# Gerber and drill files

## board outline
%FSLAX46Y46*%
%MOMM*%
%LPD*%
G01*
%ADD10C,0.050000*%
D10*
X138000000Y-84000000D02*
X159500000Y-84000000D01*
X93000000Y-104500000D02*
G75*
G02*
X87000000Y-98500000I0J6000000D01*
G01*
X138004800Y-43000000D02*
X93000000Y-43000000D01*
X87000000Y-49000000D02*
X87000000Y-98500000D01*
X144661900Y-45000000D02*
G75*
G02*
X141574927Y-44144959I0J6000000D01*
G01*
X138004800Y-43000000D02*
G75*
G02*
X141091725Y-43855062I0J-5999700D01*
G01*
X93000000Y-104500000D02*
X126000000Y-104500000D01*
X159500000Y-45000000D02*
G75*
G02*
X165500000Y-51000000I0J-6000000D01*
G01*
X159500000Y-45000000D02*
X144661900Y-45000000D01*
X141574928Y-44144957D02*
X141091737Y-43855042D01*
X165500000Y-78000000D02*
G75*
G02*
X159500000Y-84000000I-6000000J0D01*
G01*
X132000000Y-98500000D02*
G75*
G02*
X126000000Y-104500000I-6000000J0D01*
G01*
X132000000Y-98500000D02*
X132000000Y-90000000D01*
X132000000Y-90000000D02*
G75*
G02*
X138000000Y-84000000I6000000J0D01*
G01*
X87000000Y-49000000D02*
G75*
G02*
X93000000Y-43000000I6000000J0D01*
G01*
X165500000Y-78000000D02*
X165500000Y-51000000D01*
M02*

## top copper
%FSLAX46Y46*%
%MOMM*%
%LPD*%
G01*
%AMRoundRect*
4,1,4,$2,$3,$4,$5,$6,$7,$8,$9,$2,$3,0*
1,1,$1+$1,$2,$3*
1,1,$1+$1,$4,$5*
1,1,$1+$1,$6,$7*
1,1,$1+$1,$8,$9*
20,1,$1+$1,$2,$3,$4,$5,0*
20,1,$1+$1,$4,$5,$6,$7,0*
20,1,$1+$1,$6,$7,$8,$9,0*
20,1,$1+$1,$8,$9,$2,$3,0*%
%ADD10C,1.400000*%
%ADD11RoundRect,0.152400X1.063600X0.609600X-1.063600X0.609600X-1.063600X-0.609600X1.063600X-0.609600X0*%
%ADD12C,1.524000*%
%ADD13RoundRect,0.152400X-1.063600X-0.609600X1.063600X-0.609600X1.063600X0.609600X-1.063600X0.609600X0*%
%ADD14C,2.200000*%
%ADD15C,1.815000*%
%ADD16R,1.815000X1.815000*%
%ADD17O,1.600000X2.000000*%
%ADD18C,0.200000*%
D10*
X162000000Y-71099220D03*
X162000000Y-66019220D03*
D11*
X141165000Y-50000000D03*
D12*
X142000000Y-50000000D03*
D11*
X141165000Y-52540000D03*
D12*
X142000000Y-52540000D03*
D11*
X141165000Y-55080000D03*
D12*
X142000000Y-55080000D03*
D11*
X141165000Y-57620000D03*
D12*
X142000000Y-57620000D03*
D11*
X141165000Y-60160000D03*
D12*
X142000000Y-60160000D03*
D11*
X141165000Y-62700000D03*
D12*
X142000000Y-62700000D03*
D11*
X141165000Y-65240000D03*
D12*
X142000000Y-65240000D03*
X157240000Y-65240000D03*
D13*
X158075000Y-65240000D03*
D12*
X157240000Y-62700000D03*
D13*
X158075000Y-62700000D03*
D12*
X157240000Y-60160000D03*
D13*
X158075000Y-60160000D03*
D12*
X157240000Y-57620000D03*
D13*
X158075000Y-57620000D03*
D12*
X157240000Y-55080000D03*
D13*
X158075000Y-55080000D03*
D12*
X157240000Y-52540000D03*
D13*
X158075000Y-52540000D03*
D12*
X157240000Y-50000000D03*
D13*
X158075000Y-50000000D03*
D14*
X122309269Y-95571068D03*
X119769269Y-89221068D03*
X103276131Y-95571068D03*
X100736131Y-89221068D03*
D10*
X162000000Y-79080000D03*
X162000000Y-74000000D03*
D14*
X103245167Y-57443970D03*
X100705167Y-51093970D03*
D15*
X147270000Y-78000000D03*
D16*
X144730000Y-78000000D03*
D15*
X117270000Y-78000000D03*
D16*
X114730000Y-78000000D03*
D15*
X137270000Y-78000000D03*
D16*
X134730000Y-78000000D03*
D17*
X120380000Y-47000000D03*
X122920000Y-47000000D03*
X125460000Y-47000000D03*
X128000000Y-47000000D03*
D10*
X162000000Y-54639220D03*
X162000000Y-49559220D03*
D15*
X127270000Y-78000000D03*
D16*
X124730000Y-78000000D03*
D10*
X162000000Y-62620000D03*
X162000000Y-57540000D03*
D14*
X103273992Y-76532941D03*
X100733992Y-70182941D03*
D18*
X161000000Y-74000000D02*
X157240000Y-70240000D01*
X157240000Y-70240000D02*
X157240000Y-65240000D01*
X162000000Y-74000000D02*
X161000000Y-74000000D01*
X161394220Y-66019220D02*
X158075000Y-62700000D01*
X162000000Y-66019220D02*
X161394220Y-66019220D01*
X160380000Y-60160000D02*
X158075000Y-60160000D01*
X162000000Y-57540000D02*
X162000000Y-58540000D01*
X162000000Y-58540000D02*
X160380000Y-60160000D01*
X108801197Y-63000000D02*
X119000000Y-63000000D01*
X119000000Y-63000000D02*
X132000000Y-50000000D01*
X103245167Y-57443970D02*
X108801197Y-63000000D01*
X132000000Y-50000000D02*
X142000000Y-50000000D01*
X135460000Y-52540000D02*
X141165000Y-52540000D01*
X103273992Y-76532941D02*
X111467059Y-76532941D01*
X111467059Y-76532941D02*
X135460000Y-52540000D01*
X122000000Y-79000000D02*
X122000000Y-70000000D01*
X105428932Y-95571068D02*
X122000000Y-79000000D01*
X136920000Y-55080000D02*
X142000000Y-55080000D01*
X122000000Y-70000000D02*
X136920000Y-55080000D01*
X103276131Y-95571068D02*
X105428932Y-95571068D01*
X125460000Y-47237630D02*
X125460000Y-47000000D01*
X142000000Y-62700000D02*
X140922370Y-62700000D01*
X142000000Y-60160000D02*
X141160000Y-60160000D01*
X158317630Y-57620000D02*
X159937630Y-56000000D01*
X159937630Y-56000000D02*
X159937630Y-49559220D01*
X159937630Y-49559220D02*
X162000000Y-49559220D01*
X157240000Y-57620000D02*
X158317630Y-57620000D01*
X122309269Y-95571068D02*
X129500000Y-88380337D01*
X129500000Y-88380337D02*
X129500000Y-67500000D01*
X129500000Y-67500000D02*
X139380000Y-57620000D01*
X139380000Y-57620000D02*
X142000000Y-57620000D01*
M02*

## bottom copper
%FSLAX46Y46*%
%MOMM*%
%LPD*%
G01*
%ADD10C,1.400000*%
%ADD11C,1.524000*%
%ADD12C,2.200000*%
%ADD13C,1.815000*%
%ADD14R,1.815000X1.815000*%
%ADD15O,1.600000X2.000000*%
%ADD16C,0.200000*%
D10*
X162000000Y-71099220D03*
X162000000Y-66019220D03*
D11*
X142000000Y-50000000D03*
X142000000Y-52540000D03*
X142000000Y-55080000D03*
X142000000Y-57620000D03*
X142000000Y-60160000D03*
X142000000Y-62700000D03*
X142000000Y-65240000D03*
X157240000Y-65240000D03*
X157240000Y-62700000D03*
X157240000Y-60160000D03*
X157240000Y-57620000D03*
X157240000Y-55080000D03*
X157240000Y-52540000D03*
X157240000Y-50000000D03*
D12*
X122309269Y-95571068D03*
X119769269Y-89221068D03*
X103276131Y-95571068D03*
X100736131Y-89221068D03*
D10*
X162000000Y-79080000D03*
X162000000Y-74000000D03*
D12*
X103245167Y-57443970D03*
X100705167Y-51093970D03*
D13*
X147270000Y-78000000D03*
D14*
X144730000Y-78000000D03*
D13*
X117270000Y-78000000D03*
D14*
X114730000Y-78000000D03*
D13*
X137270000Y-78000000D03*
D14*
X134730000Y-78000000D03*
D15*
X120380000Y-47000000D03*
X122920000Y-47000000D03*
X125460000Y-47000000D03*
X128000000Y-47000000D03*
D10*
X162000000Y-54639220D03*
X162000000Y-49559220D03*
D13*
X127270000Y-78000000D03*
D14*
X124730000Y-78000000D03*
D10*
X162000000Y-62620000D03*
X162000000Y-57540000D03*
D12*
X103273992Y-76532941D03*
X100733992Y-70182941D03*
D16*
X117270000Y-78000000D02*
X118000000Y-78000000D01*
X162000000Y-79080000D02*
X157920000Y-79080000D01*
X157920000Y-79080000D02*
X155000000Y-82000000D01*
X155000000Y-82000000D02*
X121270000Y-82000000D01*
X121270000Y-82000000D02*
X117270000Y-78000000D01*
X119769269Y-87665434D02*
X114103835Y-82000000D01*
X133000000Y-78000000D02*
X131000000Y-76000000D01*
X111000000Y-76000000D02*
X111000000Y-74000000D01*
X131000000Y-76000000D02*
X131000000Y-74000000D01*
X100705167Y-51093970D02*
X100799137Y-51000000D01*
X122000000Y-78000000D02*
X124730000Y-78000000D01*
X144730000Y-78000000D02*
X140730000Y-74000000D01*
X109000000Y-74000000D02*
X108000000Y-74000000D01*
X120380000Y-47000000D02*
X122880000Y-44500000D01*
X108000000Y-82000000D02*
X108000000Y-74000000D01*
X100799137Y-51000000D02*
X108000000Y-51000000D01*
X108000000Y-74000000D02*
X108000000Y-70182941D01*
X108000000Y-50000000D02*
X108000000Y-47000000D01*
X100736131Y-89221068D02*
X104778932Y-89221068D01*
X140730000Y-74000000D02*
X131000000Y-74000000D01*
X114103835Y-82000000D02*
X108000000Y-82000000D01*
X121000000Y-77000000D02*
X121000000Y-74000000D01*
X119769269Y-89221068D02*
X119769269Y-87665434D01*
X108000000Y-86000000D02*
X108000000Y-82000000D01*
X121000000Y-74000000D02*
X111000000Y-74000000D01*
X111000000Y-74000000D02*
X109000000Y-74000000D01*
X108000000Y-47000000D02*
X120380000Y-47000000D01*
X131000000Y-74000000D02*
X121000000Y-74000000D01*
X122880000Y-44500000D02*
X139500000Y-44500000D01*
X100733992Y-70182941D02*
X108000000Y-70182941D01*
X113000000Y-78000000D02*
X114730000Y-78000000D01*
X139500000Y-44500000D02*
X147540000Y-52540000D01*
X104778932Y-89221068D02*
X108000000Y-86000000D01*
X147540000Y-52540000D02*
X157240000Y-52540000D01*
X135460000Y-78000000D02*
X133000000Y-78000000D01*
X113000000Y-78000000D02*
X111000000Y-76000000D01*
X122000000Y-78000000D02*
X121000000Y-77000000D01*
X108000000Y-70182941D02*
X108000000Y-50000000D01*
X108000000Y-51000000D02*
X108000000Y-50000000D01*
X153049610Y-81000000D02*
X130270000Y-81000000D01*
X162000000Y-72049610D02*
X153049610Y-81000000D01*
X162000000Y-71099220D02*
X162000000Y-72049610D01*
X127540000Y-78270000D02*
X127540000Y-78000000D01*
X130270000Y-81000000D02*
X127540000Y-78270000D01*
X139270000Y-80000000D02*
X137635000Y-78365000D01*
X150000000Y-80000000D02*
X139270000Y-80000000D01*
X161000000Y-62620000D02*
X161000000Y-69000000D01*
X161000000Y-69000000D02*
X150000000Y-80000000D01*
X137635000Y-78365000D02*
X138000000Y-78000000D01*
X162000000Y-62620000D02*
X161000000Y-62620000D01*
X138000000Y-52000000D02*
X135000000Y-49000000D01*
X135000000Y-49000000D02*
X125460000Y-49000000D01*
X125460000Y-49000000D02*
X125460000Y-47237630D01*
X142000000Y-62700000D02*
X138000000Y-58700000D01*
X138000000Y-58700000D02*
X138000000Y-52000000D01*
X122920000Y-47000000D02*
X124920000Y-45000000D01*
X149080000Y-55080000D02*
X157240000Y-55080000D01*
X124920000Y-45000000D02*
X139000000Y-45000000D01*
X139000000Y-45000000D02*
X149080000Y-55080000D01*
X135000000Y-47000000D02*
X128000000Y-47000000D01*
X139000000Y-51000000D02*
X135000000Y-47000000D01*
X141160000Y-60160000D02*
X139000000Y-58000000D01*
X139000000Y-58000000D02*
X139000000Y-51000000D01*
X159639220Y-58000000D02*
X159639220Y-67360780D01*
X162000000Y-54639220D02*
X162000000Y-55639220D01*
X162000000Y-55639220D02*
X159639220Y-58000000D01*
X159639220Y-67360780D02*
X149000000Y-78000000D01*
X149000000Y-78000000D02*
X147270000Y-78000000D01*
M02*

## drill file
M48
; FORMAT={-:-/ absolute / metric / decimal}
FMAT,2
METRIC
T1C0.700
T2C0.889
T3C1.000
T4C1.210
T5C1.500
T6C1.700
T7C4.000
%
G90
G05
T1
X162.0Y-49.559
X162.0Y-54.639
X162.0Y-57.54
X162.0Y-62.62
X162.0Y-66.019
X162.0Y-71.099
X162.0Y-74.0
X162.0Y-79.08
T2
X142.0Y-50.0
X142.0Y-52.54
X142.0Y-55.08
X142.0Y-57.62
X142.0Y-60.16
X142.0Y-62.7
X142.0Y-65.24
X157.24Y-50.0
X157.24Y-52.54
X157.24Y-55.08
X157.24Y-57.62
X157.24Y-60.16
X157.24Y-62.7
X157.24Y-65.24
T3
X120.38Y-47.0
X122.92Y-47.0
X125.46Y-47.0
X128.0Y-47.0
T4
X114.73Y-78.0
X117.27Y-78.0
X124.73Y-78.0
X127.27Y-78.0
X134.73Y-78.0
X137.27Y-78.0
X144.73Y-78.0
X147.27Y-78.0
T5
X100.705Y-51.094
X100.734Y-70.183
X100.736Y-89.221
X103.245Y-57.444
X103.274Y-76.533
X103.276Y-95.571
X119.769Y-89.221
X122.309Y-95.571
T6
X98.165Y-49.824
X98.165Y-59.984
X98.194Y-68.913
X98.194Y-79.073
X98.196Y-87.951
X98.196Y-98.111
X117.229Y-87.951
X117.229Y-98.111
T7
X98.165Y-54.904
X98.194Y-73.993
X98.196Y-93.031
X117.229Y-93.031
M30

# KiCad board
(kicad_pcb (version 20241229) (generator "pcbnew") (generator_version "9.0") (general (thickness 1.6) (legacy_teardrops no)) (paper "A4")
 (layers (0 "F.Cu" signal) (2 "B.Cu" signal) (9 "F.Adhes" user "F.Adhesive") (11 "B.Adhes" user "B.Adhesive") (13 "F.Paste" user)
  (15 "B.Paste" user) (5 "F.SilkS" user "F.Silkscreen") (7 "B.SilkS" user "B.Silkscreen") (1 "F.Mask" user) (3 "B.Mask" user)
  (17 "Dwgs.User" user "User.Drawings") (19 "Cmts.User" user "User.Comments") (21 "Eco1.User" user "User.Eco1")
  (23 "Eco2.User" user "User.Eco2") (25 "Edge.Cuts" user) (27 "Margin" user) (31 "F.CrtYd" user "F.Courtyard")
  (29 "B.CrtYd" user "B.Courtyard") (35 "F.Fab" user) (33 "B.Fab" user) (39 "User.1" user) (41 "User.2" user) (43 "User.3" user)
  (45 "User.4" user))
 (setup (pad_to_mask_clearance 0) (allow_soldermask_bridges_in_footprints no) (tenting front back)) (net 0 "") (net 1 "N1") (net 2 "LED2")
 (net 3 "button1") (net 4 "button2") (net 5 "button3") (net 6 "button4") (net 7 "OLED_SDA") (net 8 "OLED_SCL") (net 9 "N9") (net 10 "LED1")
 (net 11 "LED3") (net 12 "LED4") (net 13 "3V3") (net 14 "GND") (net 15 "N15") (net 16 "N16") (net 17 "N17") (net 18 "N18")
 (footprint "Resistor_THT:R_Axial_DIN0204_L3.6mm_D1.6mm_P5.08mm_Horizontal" (layer "F.Cu") (at 162 71.09922 90)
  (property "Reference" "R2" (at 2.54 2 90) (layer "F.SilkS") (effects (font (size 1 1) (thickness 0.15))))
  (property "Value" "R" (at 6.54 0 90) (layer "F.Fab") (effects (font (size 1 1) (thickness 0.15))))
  (pad "1" thru_hole circle (at 0 0 90) (size 1.4 1.4) (drill 0.7) (layers "*.Cu" "*.Mask") (remove_unused_layers no) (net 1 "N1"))
  (pad "2" thru_hole circle (at 5.08 0 90) (size 1.4 1.4) (drill 0.7) (layers "*.Cu" "*.Mask") (remove_unused_layers no) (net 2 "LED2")))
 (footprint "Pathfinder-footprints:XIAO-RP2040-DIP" (layer "F.Cu") (at 149.62 57.62)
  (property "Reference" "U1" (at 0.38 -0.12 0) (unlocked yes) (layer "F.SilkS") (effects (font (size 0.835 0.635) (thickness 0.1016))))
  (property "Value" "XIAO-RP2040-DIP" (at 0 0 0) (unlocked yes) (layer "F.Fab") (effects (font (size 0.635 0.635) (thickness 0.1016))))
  (pad "1" smd roundrect (at -8.455 -7.62 180) (size 2.432 1.524) (layers "F.Cu" "F.Mask") (roundrect_rratio 0.1) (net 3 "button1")
   (thermal_bridge_angle 45))
  (pad "1" thru_hole circle (at -7.62 -7.62 180) (size 1.524 1.524) (drill 0.889) (layers "*.Cu" "*.Mask") (remove_unused_layers no)
   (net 3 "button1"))
  (pad "2" smd roundrect (at -8.455 -5.08 180) (size 2.432 1.524) (layers "F.Cu" "F.Mask") (roundrect_rratio 0.1) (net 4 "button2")
   (thermal_bridge_angle 45))
  (pad "2" thru_hole circle (at -7.62 -5.08 180) (size 1.524 1.524) (drill 0.889) (layers "*.Cu" "*.Mask") (remove_unused_layers no)
   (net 4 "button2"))
  (pad "3" smd roundrect (at -8.455 -2.54 180) (size 2.432 1.524) (layers "F.Cu" "F.Mask") (roundrect_rratio 0.1) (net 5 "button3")
   (thermal_bridge_angle 45))
  (pad "3" thru_hole circle (at -7.62 -2.54 180) (size 1.524 1.524) (drill 0.889) (layers "*.Cu" "*.Mask") (remove_unused_layers no)
   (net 5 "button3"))
  (pad "4" smd roundrect (at -8.455 0 180) (size 2.432 1.524) (layers "F.Cu" "F.Mask") (roundrect_rratio 0.1) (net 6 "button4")
   (thermal_bridge_angle 45))
  (pad "4" thru_hole circle (at -7.62 0 180) (size 1.524 1.524) (drill 0.889) (layers "*.Cu" "*.Mask") (remove_unused_layers no)
   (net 6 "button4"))
  (pad "5" smd roundrect (at -8.455 2.54 180) (size 2.432 1.524) (layers "F.Cu" "F.Mask") (roundrect_rratio 0.1) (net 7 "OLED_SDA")
   (thermal_bridge_angle 45))
  (pad "5" thru_hole circle (at -7.62 2.54 180) (size 1.524 1.524) (drill 0.889) (layers "*.Cu" "*.Mask") (remove_unused_layers no)
   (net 7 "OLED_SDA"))
  (pad "6" smd roundrect (at -8.455 5.08 180) (size 2.432 1.524) (layers "F.Cu" "F.Mask") (roundrect_rratio 0.1) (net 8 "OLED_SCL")
   (thermal_bridge_angle 45))
  (pad "6" thru_hole circle (at -7.62 5.08 180) (size 1.524 1.524) (drill 0.889) (layers "*.Cu" "*.Mask") (remove_unused_layers no)
   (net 8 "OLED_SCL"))
  (pad "7" smd roundrect (at -8.455 7.62 180) (size 2.432 1.524) (layers "F.Cu" "F.Mask") (roundrect_rratio 0.1) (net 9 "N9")
   (thermal_bridge_angle 45))
  (pad "7" thru_hole circle (at -7.62 7.62 180) (size 1.524 1.524) (drill 0.889) (layers "*.Cu" "*.Mask") (remove_unused_layers no)
   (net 9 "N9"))
  (pad "8" thru_hole circle (at 7.62 7.62) (size 1.524 1.524) (drill 0.889) (layers "*.Cu" "*.Mask") (remove_unused_layers no)
   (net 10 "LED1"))
  (pad "8" smd roundrect (at 8.455 7.62) (size 2.432 1.524) (layers "F.Cu" "F.Mask") (roundrect_rratio 0.1) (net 10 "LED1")
   (thermal_bridge_angle 45))
  (pad "9" thru_hole circle (at 7.62 5.08) (size 1.524 1.524) (drill 0.889) (layers "*.Cu" "*.Mask") (remove_unused_layers no)
   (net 2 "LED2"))
  (pad "9" smd roundrect (at 8.455 5.08) (size 2.432 1.524) (layers "F.Cu" "F.Mask") (roundrect_rratio 0.1) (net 2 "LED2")
   (thermal_bridge_angle 45))
  (pad "10" thru_hole circle (at 7.62 2.54) (size 1.524 1.524) (drill 0.889) (layers "*.Cu" "*.Mask") (remove_unused_layers no)
   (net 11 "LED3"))
  (pad "10" smd roundrect (at 8.455 2.54) (size 2.432 1.524) (layers "F.Cu" "F.Mask") (roundrect_rratio 0.1) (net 11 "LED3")
   (thermal_bridge_angle 45))
  (pad "11" thru_hole circle (at 7.62 0) (size 1.524 1.524) (drill 0.889) (layers "*.Cu" "*.Mask") (remove_unused_layers no) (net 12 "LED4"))
  (pad "11" smd roundrect (at 8.455 0) (size 2.432 1.524) (layers "F.Cu" "F.Mask") (roundrect_rratio 0.1) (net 12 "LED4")
   (thermal_bridge_angle 45))
  (pad "12" thru_hole circle (at 7.62 -2.54) (size 1.524 1.524) (drill 0.889) (layers "*.Cu" "*.Mask") (remove_unused_layers no)
   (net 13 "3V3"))
  (pad "12" smd roundrect (at 8.455 -2.54) (size 2.432 1.524) (layers "F.Cu" "F.Mask") (roundrect_rratio 0.1) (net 13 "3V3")
   (thermal_bridge_angle 45))
  (pad "13" thru_hole circle (at 7.62 -5.08) (size 1.524 1.524) (drill 0.889) (layers "*.Cu" "*.Mask") (remove_unused_layers no)
   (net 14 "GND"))
  (pad "13" smd roundrect (at 8.455 -5.08) (size 2.432 1.524) (layers "F.Cu" "F.Mask") (roundrect_rratio 0.1) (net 14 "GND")
   (thermal_bridge_angle 45))
  (pad "14" thru_hole circle (at 7.62 -7.62) (size 1.524 1.524) (drill 0.889) (layers "*.Cu" "*.Mask") (remove_unused_layers no)
   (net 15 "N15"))
  (pad "14" smd roundrect (at 8.455 -7.62) (size 2.432 1.524) (layers "F.Cu" "F.Mask") (roundrect_rratio 0.1) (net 15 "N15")
   (thermal_bridge_angle 45)))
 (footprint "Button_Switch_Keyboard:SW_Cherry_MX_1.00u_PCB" (layer "F.Cu") (at 122.309269 95.571068 -90)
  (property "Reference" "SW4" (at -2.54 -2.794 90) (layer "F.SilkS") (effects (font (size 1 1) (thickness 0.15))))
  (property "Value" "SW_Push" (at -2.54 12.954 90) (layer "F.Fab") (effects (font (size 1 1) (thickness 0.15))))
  (pad "" np_thru_hole circle (at -7.62 5.08 270) (size 1.7 1.7) (drill 1.7) (layers "*.Cu" "*.Mask"))
  (pad "" np_thru_hole circle (at -2.54 5.08 270) (size 4 4) (drill 4) (layers "*.Cu" "*.Mask"))
  (pad "" np_thru_hole circle (at 2.54 5.08 270) (size 1.7 1.7) (drill 1.7) (layers "*.Cu" "*.Mask"))
  (pad "1" thru_hole circle (at 0 0 270) (size 2.2 2.2) (drill 1.5) (layers "*.Cu" "*.Mask") (remove_unused_layers no) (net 6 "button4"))
  (pad "2" thru_hole circle (at -6.35 2.54 270) (size 2.2 2.2) (drill 1.5) (layers "*.Cu" "*.Mask") (remove_unused_layers no) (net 14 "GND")))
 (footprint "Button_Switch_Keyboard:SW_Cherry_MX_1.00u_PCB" (layer "F.Cu") (at 103.276131 95.571068 -90)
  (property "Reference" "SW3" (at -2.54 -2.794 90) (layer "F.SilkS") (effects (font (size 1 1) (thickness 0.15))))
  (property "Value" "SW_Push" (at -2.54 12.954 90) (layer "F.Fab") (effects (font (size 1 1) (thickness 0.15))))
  (pad "" np_thru_hole circle (at -7.62 5.08 270) (size 1.7 1.7) (drill 1.7) (layers "*.Cu" "*.Mask"))
  (pad "" np_thru_hole circle (at -2.54 5.08 270) (size 4 4) (drill 4) (layers "*.Cu" "*.Mask"))
  (pad "" np_thru_hole circle (at 2.54 5.08 270) (size 1.7 1.7) (drill 1.7) (layers "*.Cu" "*.Mask"))
  (pad "1" thru_hole circle (at 0 0 270) (size 2.2 2.2) (drill 1.5) (layers "*.Cu" "*.Mask") (remove_unused_layers no) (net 5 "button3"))
  (pad "2" thru_hole circle (at -6.35 2.54 270) (size 2.2 2.2) (drill 1.5) (layers "*.Cu" "*.Mask") (remove_unused_layers no) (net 14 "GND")))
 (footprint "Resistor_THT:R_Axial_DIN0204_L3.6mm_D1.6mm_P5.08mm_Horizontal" (layer "F.Cu") (at 162 79.08 90)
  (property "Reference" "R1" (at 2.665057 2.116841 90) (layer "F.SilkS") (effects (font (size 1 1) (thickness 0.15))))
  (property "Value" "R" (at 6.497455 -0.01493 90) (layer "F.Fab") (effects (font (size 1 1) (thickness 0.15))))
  (pad "1" thru_hole circle (at 0 0 90) (size 1.4 1.4) (drill 0.7) (layers "*.Cu" "*.Mask") (remove_unused_layers no) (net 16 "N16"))
  (pad "2" thru_hole circle (at 5.08 0 90) (size 1.4 1.4) (drill 0.7) (layers "*.Cu" "*.Mask") (remove_unused_layers no) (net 10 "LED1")))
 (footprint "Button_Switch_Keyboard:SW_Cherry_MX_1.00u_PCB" (layer "F.Cu") (at 103.245167 57.44397 -90)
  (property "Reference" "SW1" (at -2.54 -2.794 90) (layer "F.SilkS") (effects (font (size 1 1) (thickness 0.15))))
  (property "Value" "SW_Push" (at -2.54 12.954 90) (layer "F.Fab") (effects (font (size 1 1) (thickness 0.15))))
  (pad "" np_thru_hole circle (at -7.62 5.08 270) (size 1.7 1.7) (drill 1.7) (layers "*.Cu" "*.Mask"))
  (pad "" np_thru_hole circle (at -2.54 5.08 270) (size 4 4) (drill 4) (layers "*.Cu" "*.Mask"))
  (pad "" np_thru_hole circle (at 2.54 5.08 270) (size 1.7 1.7) (drill 1.7) (layers "*.Cu" "*.Mask"))
  (pad "1" thru_hole circle (at 0 0 270) (size 2.2 2.2) (drill 1.5) (layers "*.Cu" "*.Mask") (remove_unused_layers no) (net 3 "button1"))
  (pad "2" thru_hole circle (at -6.35 2.54 270) (size 2.2 2.2) (drill 1.5) (layers "*.Cu" "*.Mask") (remove_unused_layers no) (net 14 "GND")))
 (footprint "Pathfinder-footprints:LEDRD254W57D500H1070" (layer "F.Cu") (at 146 78)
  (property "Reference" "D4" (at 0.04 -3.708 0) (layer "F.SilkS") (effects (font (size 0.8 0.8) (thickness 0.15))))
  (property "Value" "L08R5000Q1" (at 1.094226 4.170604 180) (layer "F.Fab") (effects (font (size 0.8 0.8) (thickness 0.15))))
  (pad "A" thru_hole circle (at 1.27 0) (size 1.815 1.815) (drill 1.21) (layers "*.Cu" "*.Mask") (remove_unused_layers no) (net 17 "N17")
   (solder_mask_margin 0.102))
  (pad "C" thru_hole rect (at -1.27 0) (size 1.815 1.815) (drill 1.21) (layers "*.Cu" "*.Mask") (remove_unused_layers no) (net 14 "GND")
   (solder_mask_margin 0.102)))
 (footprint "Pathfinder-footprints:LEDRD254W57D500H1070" (layer "F.Cu") (at 116 78)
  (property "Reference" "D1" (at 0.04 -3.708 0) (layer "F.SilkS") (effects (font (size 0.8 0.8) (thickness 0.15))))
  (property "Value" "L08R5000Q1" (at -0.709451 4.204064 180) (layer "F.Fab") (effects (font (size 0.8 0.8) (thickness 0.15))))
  (pad "A" thru_hole circle (at 1.27 0) (size 1.815 1.815) (drill 1.21) (layers "*.Cu" "*.Mask") (remove_unused_layers no) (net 16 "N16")
   (solder_mask_margin 0.102))
  (pad "C" thru_hole rect (at -1.27 0) (size 1.815 1.815) (drill 1.21) (layers "*.Cu" "*.Mask") (remove_unused_layers no) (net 14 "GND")
   (solder_mask_margin 0.102)))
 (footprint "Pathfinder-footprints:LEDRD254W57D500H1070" (layer "F.Cu") (at 136 78)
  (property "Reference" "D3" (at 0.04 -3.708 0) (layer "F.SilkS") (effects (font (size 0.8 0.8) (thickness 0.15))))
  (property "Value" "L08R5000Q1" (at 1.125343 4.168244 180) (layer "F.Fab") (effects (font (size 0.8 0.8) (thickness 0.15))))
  (pad "A" thru_hole circle (at 1.27 0) (size 1.815 1.815) (drill 1.21) (layers "*.Cu" "*.Mask") (remove_unused_layers no) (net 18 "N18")
   (solder_mask_margin 0.102))
  (pad "C" thru_hole rect (at -1.27 0) (size 1.815 1.815) (drill 1.21) (layers "*.Cu" "*.Mask") (remove_unused_layers no) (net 14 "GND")
   (solder_mask_margin 0.102)))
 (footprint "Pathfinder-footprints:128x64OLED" (layer "F.Cu") (at 124 57.6)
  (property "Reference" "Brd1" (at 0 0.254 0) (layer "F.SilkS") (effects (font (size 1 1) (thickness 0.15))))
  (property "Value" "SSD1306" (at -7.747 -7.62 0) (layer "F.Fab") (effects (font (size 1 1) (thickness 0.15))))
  (pad "1" thru_hole oval (at -3.62 -10.6 90) (size 2 1.6) (drill 1) (layers "*.Cu" "*.Mask") (remove_unused_layers no) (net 14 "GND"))
  (pad "2" thru_hole oval (at -1.08 -10.6 90) (size 2 1.6) (drill 1) (layers "*.Cu" "*.Mask") (remove_unused_layers no) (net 13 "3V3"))
  (pad "3" thru_hole oval (at 1.46 -10.6 90) (size 2 1.6) (drill 1) (layers "*.Cu" "*.Mask") (remove_unused_layers no) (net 8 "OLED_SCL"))
  (pad "4" thru_hole oval (at 4 -10.6 90) (size 2 1.6) (drill 1) (layers "*.Cu" "*.Mask") (remove_unused_layers no) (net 7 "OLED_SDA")))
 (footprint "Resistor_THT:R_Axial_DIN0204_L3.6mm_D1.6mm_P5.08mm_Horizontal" (layer "F.Cu") (at 162 54.63922 90)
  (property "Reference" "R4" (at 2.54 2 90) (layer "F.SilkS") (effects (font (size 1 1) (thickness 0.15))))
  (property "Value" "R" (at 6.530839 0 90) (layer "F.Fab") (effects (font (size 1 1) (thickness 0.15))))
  (pad "1" thru_hole circle (at 0 0 90) (size 1.4 1.4) (drill 0.7) (layers "*.Cu" "*.Mask") (remove_unused_layers no) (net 17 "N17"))
  (pad "2" thru_hole circle (at 5.08 0 90) (size 1.4 1.4) (drill 0.7) (layers "*.Cu" "*.Mask") (remove_unused_layers no) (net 12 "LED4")))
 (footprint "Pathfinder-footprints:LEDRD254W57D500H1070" (layer "F.Cu") (at 126 78)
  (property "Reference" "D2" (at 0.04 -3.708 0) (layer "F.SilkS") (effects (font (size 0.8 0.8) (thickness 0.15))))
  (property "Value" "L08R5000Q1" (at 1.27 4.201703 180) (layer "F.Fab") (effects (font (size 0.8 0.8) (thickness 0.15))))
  (pad "A" thru_hole circle (at 1.27 0) (size 1.815 1.815) (drill 1.21) (layers "*.Cu" "*.Mask") (remove_unused_layers no) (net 1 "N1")
   (solder_mask_margin 0.102))
  (pad "C" thru_hole rect (at -1.27 0) (size 1.815 1.815) (drill 1.21) (layers "*.Cu" "*.Mask") (remove_unused_layers no) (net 14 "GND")
   (solder_mask_margin 0.102)))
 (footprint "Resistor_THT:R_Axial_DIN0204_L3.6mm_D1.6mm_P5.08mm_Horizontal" (layer "F.Cu") (at 162 62.62 90)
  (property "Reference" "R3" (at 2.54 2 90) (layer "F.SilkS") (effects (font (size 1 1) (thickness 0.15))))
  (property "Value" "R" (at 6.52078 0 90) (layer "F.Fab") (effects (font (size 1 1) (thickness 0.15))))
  (pad "1" thru_hole circle (at 0 0 90) (size 1.4 1.4) (drill 0.7) (layers "*.Cu" "*.Mask") (remove_unused_layers no) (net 18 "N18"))
  (pad "2" thru_hole circle (at 5.08 0 90) (size 1.4 1.4) (drill 0.7) (layers "*.Cu" "*.Mask") (remove_unused_layers no) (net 11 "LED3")))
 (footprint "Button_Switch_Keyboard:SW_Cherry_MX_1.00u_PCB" (layer "F.Cu") (at 103.273992 76.532941 -90)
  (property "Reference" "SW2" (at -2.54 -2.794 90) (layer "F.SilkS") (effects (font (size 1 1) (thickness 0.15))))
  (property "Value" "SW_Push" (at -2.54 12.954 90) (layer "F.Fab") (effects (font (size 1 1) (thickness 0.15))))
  (pad "" np_thru_hole circle (at -7.62 5.08 270) (size 1.7 1.7) (drill 1.7) (layers "*.Cu" "*.Mask"))
  (pad "" np_thru_hole circle (at -2.54 5.08 270) (size 4 4) (drill 4) (layers "*.Cu" "*.Mask"))
  (pad "" np_thru_hole circle (at 2.54 5.08 270) (size 1.7 1.7) (drill 1.7) (layers "*.Cu" "*.Mask"))
  (pad "1" thru_hole circle (at 0 0 270) (size 2.2 2.2) (drill 1.5) (layers "*.Cu" "*.Mask") (remove_unused_layers no) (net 4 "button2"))
  (pad "2" thru_hole circle (at -6.35 2.54 270) (size 2.2 2.2) (drill 1.5) (layers "*.Cu" "*.Mask") (remove_unused_layers no) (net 14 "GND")))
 (gr_line (start 138 84) (end 159.5 84) (stroke (width 0.05) (type solid)) (layer "Edge.Cuts"))
 (gr_arc (start 93 104.5) (mid 88.757359 102.742641) (end 87 98.5) (stroke (width 0.05) (type default)) (layer "Edge.Cuts"))
 (gr_line (start 138.0048 43) (end 93 43) (stroke (width 0.05) (type default)) (layer "Edge.Cuts"))
 (gr_line (start 87 49) (end 87 98.5) (stroke (width 0.05) (type default)) (layer "Edge.Cuts"))
 (gr_arc (start 144.6619 45) (mid 143.060302 44.782289) (end 141.574928 44.144957) (stroke (width 0.05) (type default)) (layer "Edge.Cuts"))
 (gr_arc (start 138.0048 43) (mid 139.606368 43.217701) (end 141.091737 43.855042) (stroke (width 0.05) (type default)) (layer "Edge.Cuts"))
 (gr_line (start 93 104.5) (end 126 104.5) (stroke (width 0.05) (type default)) (layer "Edge.Cuts"))
 (gr_arc (start 159.5 45) (mid 163.742641 46.757359) (end 165.5 51) (stroke (width 0.05) (type default)) (layer "Edge.Cuts"))
 (gr_line (start 159.5 45) (end 144.6619 45) (stroke (width 0.05) (type default)) (layer "Edge.Cuts"))
 (gr_line (start 141.574928 44.144957) (end 141.091737 43.855042) (stroke (width 0.05) (type default)) (layer "Edge.Cuts"))
 (gr_arc (start 165.5 78) (mid 163.742641 82.242641) (end 159.5 84) (stroke (width 0.05) (type default)) (layer "Edge.Cuts"))
 (gr_arc (start 132 98.5) (mid 130.242641 102.742641) (end 126 104.5) (stroke (width 0.05) (type default)) (layer "Edge.Cuts"))
 (gr_line (start 132 98.5) (end 132 90) (stroke (width 0.05) (type default)) (layer "Edge.Cuts"))
 (gr_arc (start 132 90) (mid 133.757359 85.757359) (end 138 84) (stroke (width 0.05) (type default)) (layer "Edge.Cuts"))
 (gr_arc (start 87 49) (mid 88.757359 44.757359) (end 93 43) (stroke (width 0.05) (type default)) (layer "Edge.Cuts"))
 (gr_line (start 165.5 78) (end 165.5 51) (stroke (width 0.05) (type default)) (layer "Edge.Cuts"))
 (segment (start 117.27 78) (end 118 78) (width 0.2) (layer "B.Cu") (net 16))
 (segment (start 162 79.08) (end 157.92 79.08) (width 0.2) (layer "B.Cu") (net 16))
 (segment (start 157.92 79.08) (end 155 82) (width 0.2) (layer "B.Cu") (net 16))
 (segment (start 155 82) (end 121.27 82) (width 0.2) (layer "B.Cu") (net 16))
 (segment (start 121.27 82) (end 117.27 78) (width 0.2) (layer "B.Cu") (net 16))
 (segment (start 119.769269 87.665434) (end 114.103835 82) (width 0.2) (layer "B.Cu") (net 14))
 (segment (start 133 78) (end 131 76) (width 0.2) (layer "B.Cu") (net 14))
 (segment (start 111 76) (end 111 74) (width 0.2) (layer "B.Cu") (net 14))
 (segment (start 131 76) (end 131 74) (width 0.2) (layer "B.Cu") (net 14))
 (segment (start 100.705167 51.09397) (end 100.799137 51) (width 0.2) (layer "B.Cu") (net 14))
 (segment (start 122 78) (end 124.73 78) (width 0.2) (layer "B.Cu") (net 14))
 (segment (start 144.73 78) (end 140.73 74) (width 0.2) (layer "B.Cu") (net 14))
 (segment (start 109 74) (end 108 74) (width 0.2) (layer "B.Cu") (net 14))
 (segment (start 120.38 47) (end 122.88 44.5) (width 0.2) (layer "B.Cu") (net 14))
 (segment (start 108 82) (end 108 74) (width 0.2) (layer "B.Cu") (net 14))
 (segment (start 100.799137 51) (end 108 51) (width 0.2) (layer "B.Cu") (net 14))
 (segment (start 108 74) (end 108 70.182941) (width 0.2) (layer "B.Cu") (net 14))
 (segment (start 108 50) (end 108 47) (width 0.2) (layer "B.Cu") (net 14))
 (segment (start 100.736131 89.221068) (end 104.778932 89.221068) (width 0.2) (layer "B.Cu") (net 14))
 (segment (start 140.73 74) (end 131 74) (width 0.2) (layer "B.Cu") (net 14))
 (segment (start 114.103835 82) (end 108 82) (width 0.2) (layer "B.Cu") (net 14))
 (segment (start 121 77) (end 121 74) (width 0.2) (layer "B.Cu") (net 14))
 (segment (start 119.769269 89.221068) (end 119.769269 87.665434) (width 0.2) (layer "B.Cu") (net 14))
 (segment (start 108 86) (end 108 82) (width 0.2) (layer "B.Cu") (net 14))
 (segment (start 121 74) (end 111 74) (width 0.2) (layer "B.Cu") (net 14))
 (segment (start 111 74) (end 109 74) (width 0.2) (layer "B.Cu") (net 14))
 (segment (start 108 47) (end 120.38 47) (width 0.2) (layer "B.Cu") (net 14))
 (segment (start 131 74) (end 121 74) (width 0.2) (layer "B.Cu") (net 14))
 (segment (start 122.88 44.5) (end 139.5 44.5) (width 0.2) (layer "B.Cu") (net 14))
 (segment (start 100.733992 70.182941) (end 108 70.182941) (width 0.2) (layer "B.Cu") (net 14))
 (segment (start 113 78) (end 114.73 78) (width 0.2) (layer "B.Cu") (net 14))
 (segment (start 139.5 44.5) (end 147.54 52.54) (width 0.2) (layer "B.Cu") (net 14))
 (segment (start 104.778932 89.221068) (end 108 86) (width 0.2) (layer "B.Cu") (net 14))
 (segment (start 147.54 52.54) (end 157.24 52.54) (width 0.2) (layer "B.Cu") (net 14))
 (segment (start 135.46 78) (end 133 78) (width 0.2) (layer "B.Cu") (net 14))
 (segment (start 113 78) (end 111 76) (width 0.2) (layer "B.Cu") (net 14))
 (segment (start 122 78) (end 121 77) (width 0.2) (layer "B.Cu") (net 14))
 (segment (start 108 70.182941) (end 108 50) (width 0.2) (layer "B.Cu") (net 14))
 (segment (start 108 51) (end 108 50) (width 0.2) (layer "B.Cu") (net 14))
 (segment (start 153.04961 81) (end 130.27 81) (width 0.2) (layer "B.Cu") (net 1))
 (segment (start 162 72.04961) (end 153.04961 81) (width 0.2) (layer "B.Cu") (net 1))
 (segment (start 162 71.09922) (end 162 72.04961) (width 0.2) (layer "B.Cu") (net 1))
 (segment (start 127.54 78.27) (end 127.54 78) (width 0.2) (layer "B.Cu") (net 1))
 (segment (start 130.27 81) (end 127.54 78.27) (width 0.2) (layer "B.Cu") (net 1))
 (segment (start 139.27 80) (end 137.635 78.365) (width 0.2) (layer "B.Cu") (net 18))
 (segment (start 150 80) (end 139.27 80) (width 0.2) (layer "B.Cu") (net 18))
 (segment (start 161 62.62) (end 161 69) (width 0.2) (layer "B.Cu") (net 18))
 (segment (start 161 69) (end 150 80) (width 0.2) (layer "B.Cu") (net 18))
 (segment (start 137.635 78.365) (end 138 78) (width 0.2) (layer "B.Cu") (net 18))
 (segment (start 162 62.62) (end 161 62.62) (width 0.2) (layer "B.Cu") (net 18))
 (segment (start 161 74) (end 157.24 70.24) (width 0.2) (layer "F.Cu") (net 10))
 (segment (start 157.24 70.24) (end 157.24 65.24) (width 0.2) (layer "F.Cu") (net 10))
 (segment (start 162 74) (end 161 74) (width 0.2) (layer "F.Cu") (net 10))
 (segment (start 161.39422 66.01922) (end 158.075 62.7) (width 0.2) (layer "F.Cu") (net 2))
 (segment (start 162 66.01922) (end 161.39422 66.01922) (width 0.2) (layer "F.Cu") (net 2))
 (segment (start 160.38 60.16) (end 158.075 60.16) (width 0.2) (layer "F.Cu") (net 11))
 (segment (start 162 57.54) (end 162 58.54) (width 0.2) (layer "F.Cu") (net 11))
 (segment (start 162 58.54) (end 160.38 60.16) (width 0.2) (layer "F.Cu") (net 11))
 (segment (start 108.801197 63) (end 119 63) (width 0.2) (layer "F.Cu") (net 3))
 (segment (start 119 63) (end 132 50) (width 0.2) (layer "F.Cu") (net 3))
 (segment (start 103.245167 57.44397) (end 108.801197 63) (width 0.2) (layer "F.Cu") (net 3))
 (segment (start 132 50) (end 142 50) (width 0.2) (layer "F.Cu") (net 3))
 (segment (start 135.46 52.54) (end 141.165 52.54) (width 0.2) (layer "F.Cu") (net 4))
 (segment (start 103.273992 76.532941) (end 111.467059 76.532941) (width 0.2) (layer "F.Cu") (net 4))
 (segment (start 111.467059 76.532941) (end 135.46 52.54) (width 0.2) (layer "F.Cu") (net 4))
 (segment (start 122 79) (end 122 70) (width 0.2) (layer "F.Cu") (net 5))
 (segment (start 105.428932 95.571068) (end 122 79) (width 0.2) (layer "F.Cu") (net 5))
 (segment (start 136.92 55.08) (end 142 55.08) (width 0.2) (layer "F.Cu") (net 5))
 (segment (start 122 70) (end 136.92 55.08) (width 0.2) (layer "F.Cu") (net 5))
 (segment (start 103.276131 95.571068) (end 105.428932 95.571068) (width 0.2) (layer "F.Cu") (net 5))
 (segment (start 125.46 47.23763) (end 125.46 47) (width 0.2) (layer "F.Cu") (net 8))
 (segment (start 142 62.7) (end 140.92237 62.7) (width 0.2) (layer "F.Cu") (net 8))
 (segment (start 138 52) (end 135 49) (width 0.2) (layer "B.Cu") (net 8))
 (segment (start 135 49) (end 125.46 49) (width 0.2) (layer "B.Cu") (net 8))
 (segment (start 125.46 49) (end 125.46 47.23763) (width 0.2) (layer "B.Cu") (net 8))
 (segment (start 142 62.7) (end 138 58.7) (width 0.2) (layer "B.Cu") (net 8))
 (segment (start 138 58.7) (end 138 52) (width 0.2) (layer "B.Cu") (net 8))
 (segment (start 122.92 47) (end 124.92 45) (width 0.2) (layer "B.Cu") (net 13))
 (segment (start 149.08 55.08) (end 157.24 55.08) (width 0.2) (layer "B.Cu") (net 13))
 (segment (start 124.92 45) (end 139 45) (width 0.2) (layer "B.Cu") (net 13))
 (segment (start 139 45) (end 149.08 55.08) (width 0.2) (layer "B.Cu") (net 13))
 (segment (start 142 60.16) (end 141.16 60.16) (width 0.2) (layer "F.Cu") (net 7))
 (segment (start 135 47) (end 128 47) (width 0.2) (layer "B.Cu") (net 7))
 (segment (start 139 51) (end 135 47) (width 0.2) (layer "B.Cu") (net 7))
 (segment (start 141.16 60.16) (end 139 58) (width 0.2) (layer "B.Cu") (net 7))
 (segment (start 139 58) (end 139 51) (width 0.2) (layer "B.Cu") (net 7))
 (segment (start 159.63922 58) (end 159.63922 67.36078) (width 0.2) (layer "B.Cu") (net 17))
 (segment (start 162 54.63922) (end 162 55.63922) (width 0.2) (layer "B.Cu") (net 17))
 (segment (start 162 55.63922) (end 159.63922 58) (width 0.2) (layer "B.Cu") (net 17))
 (segment (start 159.63922 67.36078) (end 149 78) (width 0.2) (layer "B.Cu") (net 17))
 (segment (start 149 78) (end 147.27 78) (width 0.2) (layer "B.Cu") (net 17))
 (segment (start 158.31763 57.62) (end 159.93763 56) (width 0.2) (layer "F.Cu") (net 12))
 (segment (start 159.93763 56) (end 159.93763 49.55922) (width 0.2) (layer "F.Cu") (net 12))
 (segment (start 159.93763 49.55922) (end 162 49.55922) (width 0.2) (layer "F.Cu") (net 12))
 (segment (start 157.24 57.62) (end 158.31763 57.62) (width 0.2) (layer "F.Cu") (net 12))
 (segment (start 122.309269 95.571068) (end 129.5 88.380337) (width 0.2) (layer "F.Cu") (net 6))
 (segment (start 129.5 88.380337) (end 129.5 67.5) (width 0.2) (layer "F.Cu") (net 6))
 (segment (start 129.5 67.5) (end 139.38 57.62) (width 0.2) (layer "F.Cu") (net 6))
 (segment (start 139.38 57.62) (end 142 57.62) (width 0.2) (layer "F.Cu") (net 6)))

